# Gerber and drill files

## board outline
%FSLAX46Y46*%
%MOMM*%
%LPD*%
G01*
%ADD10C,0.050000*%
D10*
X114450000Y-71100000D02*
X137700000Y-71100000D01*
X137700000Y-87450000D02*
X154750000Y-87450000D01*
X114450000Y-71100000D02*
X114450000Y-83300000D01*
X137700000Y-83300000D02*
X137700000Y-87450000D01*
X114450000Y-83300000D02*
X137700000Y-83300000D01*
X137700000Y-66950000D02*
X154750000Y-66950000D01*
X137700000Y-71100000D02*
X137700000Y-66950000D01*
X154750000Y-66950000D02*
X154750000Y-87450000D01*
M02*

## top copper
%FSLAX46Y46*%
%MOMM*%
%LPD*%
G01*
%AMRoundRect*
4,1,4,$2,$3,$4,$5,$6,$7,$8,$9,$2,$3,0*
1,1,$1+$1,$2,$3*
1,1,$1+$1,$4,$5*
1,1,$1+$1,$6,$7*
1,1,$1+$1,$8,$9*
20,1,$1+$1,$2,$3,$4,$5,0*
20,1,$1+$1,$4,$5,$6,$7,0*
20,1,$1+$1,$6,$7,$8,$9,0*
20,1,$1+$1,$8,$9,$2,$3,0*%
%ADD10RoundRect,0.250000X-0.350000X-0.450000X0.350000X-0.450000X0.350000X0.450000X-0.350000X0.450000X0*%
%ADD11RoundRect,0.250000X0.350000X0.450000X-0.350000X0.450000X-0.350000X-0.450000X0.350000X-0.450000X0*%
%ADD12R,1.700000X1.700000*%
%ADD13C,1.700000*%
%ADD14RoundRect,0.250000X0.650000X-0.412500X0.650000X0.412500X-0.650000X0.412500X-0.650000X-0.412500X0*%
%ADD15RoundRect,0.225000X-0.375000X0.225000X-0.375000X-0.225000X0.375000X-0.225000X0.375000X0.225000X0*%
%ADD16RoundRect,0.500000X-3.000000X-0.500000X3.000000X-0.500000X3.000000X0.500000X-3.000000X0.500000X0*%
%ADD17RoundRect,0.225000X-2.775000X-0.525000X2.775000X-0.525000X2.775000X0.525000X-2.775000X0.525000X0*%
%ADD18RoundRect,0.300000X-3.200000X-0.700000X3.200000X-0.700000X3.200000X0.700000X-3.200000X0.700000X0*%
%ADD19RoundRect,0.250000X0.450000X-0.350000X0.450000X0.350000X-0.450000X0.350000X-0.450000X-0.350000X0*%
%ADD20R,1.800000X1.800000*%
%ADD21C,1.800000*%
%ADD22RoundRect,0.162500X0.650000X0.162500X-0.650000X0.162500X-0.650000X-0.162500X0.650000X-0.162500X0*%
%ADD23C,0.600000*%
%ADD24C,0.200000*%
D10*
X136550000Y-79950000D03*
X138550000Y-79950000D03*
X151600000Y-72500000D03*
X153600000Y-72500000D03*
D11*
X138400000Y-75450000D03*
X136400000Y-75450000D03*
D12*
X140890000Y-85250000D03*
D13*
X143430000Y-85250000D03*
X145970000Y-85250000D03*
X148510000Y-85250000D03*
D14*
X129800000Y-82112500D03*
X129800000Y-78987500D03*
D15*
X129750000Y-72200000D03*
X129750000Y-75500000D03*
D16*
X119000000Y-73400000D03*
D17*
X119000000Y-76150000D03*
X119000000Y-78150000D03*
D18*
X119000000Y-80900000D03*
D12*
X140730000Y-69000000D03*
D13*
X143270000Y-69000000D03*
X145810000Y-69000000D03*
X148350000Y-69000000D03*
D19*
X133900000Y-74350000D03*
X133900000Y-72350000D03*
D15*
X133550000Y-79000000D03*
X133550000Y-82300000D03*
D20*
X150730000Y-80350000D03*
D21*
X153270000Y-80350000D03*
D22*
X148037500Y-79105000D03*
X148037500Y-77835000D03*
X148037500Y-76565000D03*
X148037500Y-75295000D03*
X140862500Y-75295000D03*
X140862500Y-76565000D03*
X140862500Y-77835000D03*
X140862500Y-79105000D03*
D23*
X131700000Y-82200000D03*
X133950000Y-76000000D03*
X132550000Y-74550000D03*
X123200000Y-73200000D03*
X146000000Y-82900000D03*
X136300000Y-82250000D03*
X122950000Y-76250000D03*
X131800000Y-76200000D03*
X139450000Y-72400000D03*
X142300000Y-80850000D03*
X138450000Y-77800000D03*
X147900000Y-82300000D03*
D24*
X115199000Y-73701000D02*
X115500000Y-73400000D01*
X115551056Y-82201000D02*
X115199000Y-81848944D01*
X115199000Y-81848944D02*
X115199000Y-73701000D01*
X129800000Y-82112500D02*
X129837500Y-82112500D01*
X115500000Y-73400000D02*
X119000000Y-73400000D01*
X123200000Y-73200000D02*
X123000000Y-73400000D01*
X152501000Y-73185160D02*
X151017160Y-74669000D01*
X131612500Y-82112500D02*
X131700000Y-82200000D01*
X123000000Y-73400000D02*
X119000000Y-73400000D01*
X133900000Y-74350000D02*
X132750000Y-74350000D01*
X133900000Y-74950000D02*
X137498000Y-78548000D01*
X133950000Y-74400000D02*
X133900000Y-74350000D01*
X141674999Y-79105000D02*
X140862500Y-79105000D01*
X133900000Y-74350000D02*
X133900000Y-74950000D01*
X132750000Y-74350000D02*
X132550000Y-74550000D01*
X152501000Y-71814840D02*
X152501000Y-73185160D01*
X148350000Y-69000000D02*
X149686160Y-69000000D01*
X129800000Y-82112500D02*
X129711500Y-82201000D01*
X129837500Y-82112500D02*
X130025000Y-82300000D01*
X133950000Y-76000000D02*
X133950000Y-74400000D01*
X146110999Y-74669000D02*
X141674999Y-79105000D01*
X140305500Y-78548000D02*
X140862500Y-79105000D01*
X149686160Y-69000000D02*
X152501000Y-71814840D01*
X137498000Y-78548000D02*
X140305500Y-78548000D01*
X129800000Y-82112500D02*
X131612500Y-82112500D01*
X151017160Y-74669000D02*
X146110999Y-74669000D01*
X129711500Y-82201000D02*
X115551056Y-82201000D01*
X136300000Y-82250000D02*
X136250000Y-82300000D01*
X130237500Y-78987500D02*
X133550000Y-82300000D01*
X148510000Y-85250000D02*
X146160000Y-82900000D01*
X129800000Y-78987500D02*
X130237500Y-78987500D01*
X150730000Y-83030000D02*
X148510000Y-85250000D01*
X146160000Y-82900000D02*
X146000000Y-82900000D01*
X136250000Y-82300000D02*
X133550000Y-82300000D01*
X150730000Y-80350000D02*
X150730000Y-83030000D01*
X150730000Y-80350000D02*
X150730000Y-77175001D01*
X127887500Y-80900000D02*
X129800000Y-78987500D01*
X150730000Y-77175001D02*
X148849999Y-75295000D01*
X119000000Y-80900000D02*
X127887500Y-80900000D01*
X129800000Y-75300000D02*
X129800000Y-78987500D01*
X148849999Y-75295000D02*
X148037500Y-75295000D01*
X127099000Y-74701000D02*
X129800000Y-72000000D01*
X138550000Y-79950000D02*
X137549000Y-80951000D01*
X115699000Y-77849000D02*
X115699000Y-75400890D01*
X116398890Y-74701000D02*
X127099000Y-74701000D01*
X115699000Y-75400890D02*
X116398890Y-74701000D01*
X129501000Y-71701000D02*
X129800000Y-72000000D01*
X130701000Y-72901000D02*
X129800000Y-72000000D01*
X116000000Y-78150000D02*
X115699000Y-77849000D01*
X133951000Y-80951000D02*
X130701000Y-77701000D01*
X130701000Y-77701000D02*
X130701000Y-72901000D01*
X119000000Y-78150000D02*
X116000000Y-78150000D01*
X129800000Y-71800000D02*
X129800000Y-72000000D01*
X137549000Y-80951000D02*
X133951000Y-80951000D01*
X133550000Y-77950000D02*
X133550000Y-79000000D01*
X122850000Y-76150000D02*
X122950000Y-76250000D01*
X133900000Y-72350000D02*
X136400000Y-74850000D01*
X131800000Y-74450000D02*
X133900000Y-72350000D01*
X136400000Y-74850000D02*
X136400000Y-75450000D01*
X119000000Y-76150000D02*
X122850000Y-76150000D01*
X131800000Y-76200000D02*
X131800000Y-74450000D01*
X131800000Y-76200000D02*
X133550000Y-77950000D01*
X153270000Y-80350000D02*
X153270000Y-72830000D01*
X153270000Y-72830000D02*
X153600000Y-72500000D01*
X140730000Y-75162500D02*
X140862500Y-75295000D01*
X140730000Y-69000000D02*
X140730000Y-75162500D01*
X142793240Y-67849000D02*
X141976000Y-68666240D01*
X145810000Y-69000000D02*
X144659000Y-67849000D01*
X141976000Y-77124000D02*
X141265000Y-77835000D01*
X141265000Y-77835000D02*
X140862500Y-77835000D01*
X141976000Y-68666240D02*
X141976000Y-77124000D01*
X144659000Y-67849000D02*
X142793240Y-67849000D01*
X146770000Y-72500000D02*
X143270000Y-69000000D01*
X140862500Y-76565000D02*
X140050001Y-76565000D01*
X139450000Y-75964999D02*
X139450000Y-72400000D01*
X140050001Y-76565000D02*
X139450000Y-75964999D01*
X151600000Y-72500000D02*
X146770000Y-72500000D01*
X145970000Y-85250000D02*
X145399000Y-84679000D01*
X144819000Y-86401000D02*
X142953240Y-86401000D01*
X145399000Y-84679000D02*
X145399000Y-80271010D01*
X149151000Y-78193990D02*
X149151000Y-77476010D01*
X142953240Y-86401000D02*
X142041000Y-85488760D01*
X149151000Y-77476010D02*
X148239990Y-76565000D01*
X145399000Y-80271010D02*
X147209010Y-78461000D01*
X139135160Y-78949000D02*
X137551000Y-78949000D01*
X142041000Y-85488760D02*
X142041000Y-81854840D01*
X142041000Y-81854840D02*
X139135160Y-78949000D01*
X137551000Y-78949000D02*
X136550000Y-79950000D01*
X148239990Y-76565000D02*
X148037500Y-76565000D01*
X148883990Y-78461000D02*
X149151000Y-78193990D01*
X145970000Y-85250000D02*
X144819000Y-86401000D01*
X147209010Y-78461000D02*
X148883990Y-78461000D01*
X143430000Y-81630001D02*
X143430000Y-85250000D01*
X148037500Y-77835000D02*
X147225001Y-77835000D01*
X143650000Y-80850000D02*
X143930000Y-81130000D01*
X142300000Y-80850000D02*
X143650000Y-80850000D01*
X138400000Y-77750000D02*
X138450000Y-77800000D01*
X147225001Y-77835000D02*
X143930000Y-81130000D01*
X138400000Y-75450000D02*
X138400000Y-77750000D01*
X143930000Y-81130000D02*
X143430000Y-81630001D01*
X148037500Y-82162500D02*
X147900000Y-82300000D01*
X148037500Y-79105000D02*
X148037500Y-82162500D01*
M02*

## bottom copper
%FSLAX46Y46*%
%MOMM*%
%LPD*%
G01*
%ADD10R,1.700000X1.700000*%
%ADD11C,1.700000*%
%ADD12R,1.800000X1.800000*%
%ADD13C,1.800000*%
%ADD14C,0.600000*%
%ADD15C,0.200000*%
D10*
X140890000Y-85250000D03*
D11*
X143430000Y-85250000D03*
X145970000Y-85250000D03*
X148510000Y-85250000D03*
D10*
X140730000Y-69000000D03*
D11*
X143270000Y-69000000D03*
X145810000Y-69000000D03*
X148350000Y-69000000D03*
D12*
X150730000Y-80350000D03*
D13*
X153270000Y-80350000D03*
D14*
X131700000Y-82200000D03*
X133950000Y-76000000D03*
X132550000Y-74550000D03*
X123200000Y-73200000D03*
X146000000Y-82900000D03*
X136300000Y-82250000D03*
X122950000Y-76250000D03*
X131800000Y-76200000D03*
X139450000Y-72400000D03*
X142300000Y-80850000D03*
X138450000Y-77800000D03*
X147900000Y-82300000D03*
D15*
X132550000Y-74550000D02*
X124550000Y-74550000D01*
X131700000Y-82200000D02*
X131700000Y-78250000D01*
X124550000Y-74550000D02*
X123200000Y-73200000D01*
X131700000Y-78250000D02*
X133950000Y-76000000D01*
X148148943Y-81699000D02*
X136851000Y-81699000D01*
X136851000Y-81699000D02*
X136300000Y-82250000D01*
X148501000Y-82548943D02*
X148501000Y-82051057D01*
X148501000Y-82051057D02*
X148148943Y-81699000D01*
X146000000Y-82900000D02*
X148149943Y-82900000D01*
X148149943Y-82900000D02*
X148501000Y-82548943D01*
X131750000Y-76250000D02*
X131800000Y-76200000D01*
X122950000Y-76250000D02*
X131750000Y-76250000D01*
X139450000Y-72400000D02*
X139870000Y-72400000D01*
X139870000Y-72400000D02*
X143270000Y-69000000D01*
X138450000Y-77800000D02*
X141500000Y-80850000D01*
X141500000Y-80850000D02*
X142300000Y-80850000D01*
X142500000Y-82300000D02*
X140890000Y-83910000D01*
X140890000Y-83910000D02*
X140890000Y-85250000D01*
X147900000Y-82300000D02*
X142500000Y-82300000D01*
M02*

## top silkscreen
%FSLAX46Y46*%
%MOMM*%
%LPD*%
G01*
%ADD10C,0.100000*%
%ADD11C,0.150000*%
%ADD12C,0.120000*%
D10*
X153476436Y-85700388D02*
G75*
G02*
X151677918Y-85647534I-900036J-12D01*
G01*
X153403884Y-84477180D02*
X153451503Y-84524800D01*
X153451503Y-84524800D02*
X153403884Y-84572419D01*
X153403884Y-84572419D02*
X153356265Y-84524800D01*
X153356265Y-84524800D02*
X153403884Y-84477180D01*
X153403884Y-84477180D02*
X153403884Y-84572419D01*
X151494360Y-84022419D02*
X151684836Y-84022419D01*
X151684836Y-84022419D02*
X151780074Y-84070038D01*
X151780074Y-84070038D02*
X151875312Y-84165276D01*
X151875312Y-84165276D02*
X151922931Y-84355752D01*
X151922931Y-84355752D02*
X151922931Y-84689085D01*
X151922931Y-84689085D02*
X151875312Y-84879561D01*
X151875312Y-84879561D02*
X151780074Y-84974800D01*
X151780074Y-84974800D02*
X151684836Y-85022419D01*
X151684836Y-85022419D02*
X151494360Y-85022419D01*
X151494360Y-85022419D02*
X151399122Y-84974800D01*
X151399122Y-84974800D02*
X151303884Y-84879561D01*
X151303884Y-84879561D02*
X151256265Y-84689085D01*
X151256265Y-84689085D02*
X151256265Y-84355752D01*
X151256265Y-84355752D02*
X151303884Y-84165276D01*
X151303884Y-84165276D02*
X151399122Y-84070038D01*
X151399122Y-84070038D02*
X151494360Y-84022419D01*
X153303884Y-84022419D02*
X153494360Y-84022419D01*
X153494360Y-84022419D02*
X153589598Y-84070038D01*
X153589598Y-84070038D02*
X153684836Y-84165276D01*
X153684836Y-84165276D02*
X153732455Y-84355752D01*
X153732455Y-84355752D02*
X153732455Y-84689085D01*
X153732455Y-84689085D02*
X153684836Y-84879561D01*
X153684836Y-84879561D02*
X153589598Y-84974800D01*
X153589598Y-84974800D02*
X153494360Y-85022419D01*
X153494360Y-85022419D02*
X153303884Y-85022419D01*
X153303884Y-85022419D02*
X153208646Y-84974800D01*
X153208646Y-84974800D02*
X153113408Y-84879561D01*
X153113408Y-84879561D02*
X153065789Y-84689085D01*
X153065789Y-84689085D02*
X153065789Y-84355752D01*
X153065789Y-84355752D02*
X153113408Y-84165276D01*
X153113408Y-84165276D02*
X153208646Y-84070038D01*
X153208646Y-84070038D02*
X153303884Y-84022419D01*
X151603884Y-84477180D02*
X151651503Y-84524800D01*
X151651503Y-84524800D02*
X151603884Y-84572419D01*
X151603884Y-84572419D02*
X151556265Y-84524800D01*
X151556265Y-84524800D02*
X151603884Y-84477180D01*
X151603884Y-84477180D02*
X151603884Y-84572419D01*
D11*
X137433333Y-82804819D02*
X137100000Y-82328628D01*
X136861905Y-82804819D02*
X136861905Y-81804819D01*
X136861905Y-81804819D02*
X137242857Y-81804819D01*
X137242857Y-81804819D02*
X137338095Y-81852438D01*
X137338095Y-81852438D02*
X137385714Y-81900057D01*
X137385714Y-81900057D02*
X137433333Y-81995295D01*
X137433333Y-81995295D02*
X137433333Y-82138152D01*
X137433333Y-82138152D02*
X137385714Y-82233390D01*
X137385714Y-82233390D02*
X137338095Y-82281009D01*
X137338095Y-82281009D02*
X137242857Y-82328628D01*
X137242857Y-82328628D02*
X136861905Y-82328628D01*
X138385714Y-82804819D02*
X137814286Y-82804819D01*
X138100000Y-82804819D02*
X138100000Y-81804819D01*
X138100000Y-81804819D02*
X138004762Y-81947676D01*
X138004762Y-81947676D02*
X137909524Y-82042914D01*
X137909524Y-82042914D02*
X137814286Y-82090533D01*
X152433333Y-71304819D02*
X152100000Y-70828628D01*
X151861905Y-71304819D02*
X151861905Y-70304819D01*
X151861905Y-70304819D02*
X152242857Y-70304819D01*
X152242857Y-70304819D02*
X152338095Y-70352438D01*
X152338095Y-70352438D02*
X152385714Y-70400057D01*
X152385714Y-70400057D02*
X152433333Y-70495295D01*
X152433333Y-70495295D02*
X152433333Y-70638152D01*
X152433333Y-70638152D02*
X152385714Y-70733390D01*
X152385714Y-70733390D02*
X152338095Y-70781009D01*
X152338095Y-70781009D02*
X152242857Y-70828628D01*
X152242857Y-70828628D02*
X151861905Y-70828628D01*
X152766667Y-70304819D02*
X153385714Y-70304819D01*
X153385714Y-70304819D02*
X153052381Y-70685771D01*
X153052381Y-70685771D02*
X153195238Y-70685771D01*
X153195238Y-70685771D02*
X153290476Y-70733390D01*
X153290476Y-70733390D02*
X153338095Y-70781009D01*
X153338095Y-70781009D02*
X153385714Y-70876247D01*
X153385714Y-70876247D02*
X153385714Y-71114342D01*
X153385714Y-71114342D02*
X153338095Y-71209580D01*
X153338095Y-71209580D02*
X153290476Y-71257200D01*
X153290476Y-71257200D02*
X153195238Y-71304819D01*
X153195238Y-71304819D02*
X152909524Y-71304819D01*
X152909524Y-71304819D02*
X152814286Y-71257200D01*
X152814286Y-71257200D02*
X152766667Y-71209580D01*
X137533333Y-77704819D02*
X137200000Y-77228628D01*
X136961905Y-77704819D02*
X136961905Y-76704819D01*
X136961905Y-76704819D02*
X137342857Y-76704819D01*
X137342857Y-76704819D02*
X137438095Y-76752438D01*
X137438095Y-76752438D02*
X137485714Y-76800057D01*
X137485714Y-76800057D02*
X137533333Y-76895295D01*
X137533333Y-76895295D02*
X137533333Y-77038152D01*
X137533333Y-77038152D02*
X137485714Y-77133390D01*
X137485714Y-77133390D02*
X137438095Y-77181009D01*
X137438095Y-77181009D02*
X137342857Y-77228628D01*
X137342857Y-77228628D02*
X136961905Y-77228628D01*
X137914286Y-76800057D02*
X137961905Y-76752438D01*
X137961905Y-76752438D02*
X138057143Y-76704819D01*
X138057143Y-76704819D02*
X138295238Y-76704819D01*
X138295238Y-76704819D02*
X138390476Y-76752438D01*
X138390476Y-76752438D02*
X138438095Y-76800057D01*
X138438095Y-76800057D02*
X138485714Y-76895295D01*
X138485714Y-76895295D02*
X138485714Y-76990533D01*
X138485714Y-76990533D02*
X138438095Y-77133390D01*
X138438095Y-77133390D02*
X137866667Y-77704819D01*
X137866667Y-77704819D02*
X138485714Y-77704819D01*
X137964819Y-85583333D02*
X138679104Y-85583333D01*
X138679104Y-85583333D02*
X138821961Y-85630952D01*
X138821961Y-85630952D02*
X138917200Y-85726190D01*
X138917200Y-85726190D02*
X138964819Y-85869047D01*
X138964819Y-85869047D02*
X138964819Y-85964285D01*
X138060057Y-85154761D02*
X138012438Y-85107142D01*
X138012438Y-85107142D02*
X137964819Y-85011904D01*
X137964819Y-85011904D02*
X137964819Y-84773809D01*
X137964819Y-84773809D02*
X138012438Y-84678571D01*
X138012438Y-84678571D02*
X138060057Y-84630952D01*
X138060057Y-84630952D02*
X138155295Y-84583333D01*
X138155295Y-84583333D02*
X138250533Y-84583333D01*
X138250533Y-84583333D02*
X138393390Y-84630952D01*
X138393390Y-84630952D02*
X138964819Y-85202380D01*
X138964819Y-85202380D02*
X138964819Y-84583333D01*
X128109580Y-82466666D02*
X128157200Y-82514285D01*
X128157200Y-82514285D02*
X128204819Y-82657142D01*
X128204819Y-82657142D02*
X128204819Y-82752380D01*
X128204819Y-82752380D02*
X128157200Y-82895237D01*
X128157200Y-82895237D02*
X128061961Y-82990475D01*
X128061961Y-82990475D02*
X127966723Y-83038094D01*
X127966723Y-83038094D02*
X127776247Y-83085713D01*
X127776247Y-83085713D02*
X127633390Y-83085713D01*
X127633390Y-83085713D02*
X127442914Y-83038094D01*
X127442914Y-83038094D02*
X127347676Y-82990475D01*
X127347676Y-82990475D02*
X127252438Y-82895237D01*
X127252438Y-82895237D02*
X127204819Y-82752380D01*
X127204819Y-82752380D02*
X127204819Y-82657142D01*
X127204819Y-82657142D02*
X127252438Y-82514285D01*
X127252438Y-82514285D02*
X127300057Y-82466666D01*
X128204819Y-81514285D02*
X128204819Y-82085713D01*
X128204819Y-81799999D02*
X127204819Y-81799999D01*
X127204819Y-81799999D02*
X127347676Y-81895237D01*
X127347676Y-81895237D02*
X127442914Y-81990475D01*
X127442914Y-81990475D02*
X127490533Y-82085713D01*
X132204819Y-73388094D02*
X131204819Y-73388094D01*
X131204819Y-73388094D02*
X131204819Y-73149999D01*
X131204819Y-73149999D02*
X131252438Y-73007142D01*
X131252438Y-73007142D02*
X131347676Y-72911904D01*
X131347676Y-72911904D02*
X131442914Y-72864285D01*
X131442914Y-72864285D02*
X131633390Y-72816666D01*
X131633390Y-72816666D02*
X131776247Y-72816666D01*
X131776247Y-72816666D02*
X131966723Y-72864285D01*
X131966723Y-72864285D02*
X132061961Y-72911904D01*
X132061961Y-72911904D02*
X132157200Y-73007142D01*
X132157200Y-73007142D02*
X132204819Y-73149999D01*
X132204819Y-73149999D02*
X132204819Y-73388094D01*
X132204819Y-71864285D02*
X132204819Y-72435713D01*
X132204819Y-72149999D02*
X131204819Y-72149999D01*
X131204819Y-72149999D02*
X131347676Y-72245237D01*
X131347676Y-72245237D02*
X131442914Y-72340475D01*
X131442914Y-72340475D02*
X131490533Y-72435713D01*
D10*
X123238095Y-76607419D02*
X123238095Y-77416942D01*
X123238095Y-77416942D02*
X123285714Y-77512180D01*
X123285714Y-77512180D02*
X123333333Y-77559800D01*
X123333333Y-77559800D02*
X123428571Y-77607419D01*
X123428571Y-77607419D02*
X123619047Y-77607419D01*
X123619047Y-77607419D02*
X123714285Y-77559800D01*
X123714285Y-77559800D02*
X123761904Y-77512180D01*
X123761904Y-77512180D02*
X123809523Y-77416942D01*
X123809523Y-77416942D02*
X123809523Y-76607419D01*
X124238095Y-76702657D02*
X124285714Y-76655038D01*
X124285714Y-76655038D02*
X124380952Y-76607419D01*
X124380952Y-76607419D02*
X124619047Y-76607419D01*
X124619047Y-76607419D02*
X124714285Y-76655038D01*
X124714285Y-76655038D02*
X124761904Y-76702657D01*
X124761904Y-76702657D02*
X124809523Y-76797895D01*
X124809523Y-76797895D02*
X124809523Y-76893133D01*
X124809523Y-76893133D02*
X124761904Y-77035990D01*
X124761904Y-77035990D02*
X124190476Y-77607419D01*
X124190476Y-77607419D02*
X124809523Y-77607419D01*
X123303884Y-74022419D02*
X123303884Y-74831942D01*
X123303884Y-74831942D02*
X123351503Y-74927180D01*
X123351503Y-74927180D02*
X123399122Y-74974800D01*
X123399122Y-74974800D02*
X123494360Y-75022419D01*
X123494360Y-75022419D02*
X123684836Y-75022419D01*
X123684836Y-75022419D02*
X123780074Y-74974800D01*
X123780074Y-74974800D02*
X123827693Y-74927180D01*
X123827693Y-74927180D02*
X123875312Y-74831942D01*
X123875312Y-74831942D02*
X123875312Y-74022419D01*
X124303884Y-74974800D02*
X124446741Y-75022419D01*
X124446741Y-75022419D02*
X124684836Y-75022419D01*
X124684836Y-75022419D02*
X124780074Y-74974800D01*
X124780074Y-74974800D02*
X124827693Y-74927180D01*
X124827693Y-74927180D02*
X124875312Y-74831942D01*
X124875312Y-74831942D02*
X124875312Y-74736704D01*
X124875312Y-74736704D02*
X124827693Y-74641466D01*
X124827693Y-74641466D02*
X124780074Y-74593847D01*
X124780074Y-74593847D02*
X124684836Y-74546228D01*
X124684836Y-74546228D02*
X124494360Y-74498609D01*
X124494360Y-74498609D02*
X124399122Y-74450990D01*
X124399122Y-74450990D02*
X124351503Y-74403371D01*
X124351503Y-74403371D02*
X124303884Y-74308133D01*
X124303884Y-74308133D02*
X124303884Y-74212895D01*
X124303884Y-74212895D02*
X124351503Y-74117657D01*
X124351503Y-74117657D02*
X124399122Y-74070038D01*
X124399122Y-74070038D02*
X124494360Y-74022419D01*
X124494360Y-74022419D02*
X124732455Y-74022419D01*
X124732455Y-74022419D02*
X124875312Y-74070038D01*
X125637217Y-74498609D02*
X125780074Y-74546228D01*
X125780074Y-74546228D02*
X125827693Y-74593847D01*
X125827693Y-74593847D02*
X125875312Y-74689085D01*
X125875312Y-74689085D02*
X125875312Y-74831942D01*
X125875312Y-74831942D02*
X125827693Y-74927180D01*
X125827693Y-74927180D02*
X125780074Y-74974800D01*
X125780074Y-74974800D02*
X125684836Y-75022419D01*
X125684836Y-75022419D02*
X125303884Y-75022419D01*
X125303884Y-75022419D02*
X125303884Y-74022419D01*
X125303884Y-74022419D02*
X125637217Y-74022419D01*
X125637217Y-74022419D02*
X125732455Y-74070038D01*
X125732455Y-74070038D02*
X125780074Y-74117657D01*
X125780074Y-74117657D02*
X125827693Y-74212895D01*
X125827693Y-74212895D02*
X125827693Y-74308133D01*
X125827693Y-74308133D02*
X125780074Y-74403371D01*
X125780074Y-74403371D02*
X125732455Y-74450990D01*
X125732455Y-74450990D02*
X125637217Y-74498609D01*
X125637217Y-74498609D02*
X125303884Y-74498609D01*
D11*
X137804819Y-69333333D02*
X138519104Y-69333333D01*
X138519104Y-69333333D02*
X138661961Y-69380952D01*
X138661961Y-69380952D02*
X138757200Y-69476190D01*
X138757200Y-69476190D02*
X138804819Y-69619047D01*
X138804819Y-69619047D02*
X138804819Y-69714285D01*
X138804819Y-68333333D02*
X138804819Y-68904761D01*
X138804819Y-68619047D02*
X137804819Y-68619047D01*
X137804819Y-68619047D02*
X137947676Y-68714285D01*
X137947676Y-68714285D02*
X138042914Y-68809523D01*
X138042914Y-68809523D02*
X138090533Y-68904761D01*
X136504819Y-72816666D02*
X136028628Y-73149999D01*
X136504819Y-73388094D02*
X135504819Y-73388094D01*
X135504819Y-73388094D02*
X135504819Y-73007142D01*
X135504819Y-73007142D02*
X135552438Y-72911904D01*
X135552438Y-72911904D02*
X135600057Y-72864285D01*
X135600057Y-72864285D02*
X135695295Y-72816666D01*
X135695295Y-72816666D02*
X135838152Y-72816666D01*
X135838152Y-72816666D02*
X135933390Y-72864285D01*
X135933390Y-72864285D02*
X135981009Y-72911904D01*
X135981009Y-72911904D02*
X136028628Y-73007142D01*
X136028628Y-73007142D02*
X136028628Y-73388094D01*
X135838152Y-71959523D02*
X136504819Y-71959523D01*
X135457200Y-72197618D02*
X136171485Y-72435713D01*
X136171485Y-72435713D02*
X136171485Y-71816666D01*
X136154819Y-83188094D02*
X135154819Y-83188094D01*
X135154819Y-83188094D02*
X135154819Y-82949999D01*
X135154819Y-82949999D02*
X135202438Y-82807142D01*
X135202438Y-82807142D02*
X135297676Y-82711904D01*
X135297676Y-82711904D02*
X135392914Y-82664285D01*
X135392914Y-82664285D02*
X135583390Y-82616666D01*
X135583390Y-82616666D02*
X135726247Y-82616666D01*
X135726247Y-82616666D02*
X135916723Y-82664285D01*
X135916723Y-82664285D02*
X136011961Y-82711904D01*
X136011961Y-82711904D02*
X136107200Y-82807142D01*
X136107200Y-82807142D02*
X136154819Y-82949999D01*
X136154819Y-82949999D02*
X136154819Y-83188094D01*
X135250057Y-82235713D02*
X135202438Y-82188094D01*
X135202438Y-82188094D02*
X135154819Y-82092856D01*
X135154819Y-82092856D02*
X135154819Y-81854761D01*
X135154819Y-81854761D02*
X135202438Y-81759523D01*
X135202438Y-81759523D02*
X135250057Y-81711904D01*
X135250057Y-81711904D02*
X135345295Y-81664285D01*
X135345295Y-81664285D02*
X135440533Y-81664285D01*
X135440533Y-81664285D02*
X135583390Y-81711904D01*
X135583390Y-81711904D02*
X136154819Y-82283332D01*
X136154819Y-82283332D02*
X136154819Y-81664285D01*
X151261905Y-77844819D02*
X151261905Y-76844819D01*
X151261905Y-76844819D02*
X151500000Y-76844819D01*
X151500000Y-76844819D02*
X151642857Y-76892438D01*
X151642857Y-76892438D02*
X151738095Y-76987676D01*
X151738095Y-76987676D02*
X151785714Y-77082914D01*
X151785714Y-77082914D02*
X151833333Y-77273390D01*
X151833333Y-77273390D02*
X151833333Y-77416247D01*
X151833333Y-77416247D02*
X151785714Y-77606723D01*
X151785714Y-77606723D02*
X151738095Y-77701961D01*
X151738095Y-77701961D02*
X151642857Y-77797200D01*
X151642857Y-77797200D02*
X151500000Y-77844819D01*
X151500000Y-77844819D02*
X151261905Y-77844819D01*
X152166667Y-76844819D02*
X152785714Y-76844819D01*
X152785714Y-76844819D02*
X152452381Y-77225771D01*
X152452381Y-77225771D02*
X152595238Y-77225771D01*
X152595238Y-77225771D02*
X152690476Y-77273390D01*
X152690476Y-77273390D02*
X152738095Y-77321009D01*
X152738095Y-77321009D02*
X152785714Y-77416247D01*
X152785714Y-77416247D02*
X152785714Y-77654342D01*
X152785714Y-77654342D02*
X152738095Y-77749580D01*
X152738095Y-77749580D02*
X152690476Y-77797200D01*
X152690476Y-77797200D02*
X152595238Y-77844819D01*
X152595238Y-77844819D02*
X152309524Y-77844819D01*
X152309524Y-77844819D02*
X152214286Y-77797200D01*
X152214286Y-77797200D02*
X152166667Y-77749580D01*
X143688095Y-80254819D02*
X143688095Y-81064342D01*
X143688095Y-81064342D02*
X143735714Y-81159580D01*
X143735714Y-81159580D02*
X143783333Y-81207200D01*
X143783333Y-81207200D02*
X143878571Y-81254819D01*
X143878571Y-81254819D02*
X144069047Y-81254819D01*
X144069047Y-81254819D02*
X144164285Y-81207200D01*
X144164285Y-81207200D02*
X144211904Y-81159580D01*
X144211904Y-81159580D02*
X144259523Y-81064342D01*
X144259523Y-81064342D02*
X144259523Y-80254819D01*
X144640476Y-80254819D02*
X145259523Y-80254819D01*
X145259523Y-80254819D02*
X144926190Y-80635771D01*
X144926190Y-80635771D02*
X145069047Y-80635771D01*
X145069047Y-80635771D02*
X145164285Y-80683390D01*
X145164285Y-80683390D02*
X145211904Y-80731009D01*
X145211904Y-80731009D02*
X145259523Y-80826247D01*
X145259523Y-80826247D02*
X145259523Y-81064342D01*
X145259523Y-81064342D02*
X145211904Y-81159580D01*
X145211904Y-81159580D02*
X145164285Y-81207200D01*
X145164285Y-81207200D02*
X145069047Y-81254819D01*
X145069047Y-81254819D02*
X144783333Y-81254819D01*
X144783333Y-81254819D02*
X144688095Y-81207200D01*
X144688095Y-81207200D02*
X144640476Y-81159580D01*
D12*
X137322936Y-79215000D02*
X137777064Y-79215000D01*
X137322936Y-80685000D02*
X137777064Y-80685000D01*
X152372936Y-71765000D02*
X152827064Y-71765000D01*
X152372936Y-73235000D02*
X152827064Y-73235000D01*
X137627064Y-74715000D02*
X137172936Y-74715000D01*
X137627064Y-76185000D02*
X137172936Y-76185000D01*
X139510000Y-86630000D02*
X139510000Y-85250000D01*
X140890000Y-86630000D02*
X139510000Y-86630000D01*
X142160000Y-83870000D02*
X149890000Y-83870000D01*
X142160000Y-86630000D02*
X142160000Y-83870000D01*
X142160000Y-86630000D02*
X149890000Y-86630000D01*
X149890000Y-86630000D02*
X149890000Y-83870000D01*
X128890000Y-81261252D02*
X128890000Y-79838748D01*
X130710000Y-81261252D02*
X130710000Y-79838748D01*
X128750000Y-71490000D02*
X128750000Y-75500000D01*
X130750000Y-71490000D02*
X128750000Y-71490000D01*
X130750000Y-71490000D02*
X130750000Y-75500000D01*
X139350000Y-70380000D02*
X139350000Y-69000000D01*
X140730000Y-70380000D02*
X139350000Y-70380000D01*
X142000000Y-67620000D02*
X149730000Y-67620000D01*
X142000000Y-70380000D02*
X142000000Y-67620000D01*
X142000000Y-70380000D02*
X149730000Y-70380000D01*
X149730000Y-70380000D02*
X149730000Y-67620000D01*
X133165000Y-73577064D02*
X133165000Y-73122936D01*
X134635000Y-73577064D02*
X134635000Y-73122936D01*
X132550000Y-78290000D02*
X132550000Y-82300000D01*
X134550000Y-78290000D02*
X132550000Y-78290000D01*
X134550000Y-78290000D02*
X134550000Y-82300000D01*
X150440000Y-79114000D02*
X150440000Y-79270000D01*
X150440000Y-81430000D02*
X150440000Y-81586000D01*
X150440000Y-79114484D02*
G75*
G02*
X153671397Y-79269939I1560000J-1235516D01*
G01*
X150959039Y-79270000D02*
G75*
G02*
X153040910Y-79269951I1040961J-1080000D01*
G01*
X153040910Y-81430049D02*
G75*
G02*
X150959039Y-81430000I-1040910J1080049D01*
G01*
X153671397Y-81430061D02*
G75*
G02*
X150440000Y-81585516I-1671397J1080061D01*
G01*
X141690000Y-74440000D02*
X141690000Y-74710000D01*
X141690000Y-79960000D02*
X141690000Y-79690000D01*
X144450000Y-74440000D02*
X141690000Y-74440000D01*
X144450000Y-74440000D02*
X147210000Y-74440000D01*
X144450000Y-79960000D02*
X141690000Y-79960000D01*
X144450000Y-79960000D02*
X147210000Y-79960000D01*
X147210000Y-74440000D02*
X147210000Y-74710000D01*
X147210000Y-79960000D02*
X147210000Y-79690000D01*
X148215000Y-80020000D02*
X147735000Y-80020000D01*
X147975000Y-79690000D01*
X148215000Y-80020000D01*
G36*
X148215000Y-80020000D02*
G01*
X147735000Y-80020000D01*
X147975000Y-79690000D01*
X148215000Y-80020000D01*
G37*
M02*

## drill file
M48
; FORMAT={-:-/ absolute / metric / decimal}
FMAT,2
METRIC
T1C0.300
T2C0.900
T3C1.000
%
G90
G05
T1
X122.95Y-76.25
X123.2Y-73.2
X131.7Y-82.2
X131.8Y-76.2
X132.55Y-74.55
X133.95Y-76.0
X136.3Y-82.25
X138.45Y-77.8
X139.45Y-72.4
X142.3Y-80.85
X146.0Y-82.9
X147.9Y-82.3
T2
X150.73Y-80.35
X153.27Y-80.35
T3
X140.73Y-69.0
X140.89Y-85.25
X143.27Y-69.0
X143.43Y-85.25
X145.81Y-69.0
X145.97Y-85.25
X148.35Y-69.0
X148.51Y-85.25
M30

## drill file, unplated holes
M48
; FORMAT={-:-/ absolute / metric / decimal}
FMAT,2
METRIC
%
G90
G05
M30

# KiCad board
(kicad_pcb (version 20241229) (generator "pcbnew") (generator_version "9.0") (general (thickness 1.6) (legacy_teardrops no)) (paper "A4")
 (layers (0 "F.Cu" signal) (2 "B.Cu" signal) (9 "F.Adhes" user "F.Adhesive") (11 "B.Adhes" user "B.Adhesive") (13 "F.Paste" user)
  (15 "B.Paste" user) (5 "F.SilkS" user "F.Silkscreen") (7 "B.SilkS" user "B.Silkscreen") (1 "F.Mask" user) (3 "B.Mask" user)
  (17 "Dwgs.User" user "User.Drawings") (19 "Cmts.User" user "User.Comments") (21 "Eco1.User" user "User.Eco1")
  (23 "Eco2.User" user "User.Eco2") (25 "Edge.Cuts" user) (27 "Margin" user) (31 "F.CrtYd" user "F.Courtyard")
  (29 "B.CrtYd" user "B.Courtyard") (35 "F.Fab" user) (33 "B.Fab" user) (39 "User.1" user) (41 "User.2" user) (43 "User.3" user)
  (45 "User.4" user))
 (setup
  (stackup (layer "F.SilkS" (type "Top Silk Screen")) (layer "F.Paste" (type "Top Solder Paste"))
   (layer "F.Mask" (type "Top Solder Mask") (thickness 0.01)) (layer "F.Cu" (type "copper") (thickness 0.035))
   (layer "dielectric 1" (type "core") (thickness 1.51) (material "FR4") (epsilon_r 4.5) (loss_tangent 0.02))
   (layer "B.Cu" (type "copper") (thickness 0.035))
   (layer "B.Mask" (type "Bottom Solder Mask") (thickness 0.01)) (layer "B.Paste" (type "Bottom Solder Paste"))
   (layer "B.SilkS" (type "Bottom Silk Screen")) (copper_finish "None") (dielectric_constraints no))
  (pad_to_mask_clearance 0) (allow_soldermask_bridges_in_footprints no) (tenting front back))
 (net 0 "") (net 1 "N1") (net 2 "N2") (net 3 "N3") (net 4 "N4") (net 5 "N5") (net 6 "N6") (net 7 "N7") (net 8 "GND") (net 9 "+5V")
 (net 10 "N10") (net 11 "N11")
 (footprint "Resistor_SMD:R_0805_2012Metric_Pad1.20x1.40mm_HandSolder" (layer "F.Cu") (at 137.55 79.95)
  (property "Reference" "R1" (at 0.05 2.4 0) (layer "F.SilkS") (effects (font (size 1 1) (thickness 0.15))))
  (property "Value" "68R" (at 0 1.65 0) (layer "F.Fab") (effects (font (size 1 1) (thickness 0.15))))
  (fp_line (start -0.227064 -0.735) (end 0.227064 -0.735) (stroke (width 0.12) (type solid)) (layer "F.SilkS"))
  (fp_line (start -0.227064 0.735) (end 0.227064 0.735) (stroke (width 0.12) (type solid)) (layer "F.SilkS"))
  (pad "1" smd roundrect (at -1 0) (size 1.2 1.4) (layers "F.Cu" "F.Mask" "F.Paste") (roundrect_rratio 0.208333) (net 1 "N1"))
  (pad "2" smd roundrect (at 1 0) (size 1.2 1.4) (layers "F.Cu" "F.Mask" "F.Paste") (roundrect_rratio 0.208333) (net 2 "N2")))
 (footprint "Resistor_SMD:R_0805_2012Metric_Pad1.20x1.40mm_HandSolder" (layer "F.Cu") (at 152.6 72.5)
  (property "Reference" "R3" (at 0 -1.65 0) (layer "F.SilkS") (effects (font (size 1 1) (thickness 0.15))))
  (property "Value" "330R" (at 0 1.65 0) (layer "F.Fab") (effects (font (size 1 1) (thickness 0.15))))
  (fp_line (start -0.227064 -0.735) (end 0.227064 -0.735) (stroke (width 0.12) (type solid)) (layer "F.SilkS"))
  (fp_line (start -0.227064 0.735) (end 0.227064 0.735) (stroke (width 0.12) (type solid)) (layer "F.SilkS"))
  (pad "1" smd roundrect (at -1 0) (size 1.2 1.4) (layers "F.Cu" "F.Mask" "F.Paste") (roundrect_rratio 0.208333) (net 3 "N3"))
  (pad "2" smd roundrect (at 1 0) (size 1.2 1.4) (layers "F.Cu" "F.Mask" "F.Paste") (roundrect_rratio 0.208333) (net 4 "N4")))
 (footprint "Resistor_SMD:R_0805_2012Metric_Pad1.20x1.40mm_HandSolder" (layer "F.Cu") (at 137.4 75.45 180)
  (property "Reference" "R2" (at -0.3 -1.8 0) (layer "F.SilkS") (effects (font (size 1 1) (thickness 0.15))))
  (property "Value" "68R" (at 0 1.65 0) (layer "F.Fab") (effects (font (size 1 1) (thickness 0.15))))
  (fp_line (start -0.227064 0.735) (end 0.227064 0.735) (stroke (width 0.12) (type solid)) (layer "F.SilkS"))
  (fp_line (start -0.227064 -0.735) (end 0.227064 -0.735) (stroke (width 0.12) (type solid)) (layer "F.SilkS"))
  (pad "1" smd roundrect (at -1 0 180) (size 1.2 1.4) (layers "F.Cu" "F.Mask" "F.Paste") (roundrect_rratio 0.208333) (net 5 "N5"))
  (pad "2" smd roundrect (at 1 0 180) (size 1.2 1.4) (layers "F.Cu" "F.Mask" "F.Paste") (roundrect_rratio 0.208333) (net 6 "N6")))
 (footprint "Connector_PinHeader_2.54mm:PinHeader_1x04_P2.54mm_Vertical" (layer "F.Cu") (at 140.89 85.25 90)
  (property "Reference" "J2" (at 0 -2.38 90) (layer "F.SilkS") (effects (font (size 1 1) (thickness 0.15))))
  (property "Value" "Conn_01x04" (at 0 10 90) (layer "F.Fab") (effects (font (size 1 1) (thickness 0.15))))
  (fp_line (start -1.38 -1.38) (end 0 -1.38) (stroke (width 0.12) (type solid)) (layer "F.SilkS"))
  (fp_line (start -1.38 0) (end -1.38 -1.38) (stroke (width 0.12) (type solid)) (layer "F.SilkS"))
  (fp_line (start 1.38 1.27) (end 1.38 9) (stroke (width 0.12) (type solid)) (layer "F.SilkS"))
  (fp_line (start -1.38 1.27) (end 1.38 1.27) (stroke (width 0.12) (type solid)) (layer "F.SilkS"))
  (fp_line (start -1.38 1.27) (end -1.38 9) (stroke (width 0.12) (type solid)) (layer "F.SilkS"))
  (fp_line (start -1.38 9) (end 1.38 9) (stroke (width 0.12) (type solid)) (layer "F.SilkS"))
  (pad "1" thru_hole rect (at 0 0 90) (size 1.7 1.7) (drill 1) (layers "*.Cu" "*.Mask") (remove_unused_layers no) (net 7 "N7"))
  (pad "2" thru_hole circle (at 0 2.54 90) (size 1.7 1.7) (drill 1) (layers "*.Cu" "*.Mask") (remove_unused_layers no) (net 5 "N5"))
  (pad "3" thru_hole circle (at 0 5.08 90) (size 1.7 1.7) (drill 1) (layers "*.Cu" "*.Mask") (remove_unused_layers no) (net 1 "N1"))
  (pad "4" thru_hole circle (at 0 7.62 90) (size 1.7 1.7) (drill 1) (layers "*.Cu" "*.Mask") (remove_unused_layers no) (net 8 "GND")))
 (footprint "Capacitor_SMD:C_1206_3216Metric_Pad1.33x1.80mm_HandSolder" (layer "F.Cu") (at 129.8 80.55 90)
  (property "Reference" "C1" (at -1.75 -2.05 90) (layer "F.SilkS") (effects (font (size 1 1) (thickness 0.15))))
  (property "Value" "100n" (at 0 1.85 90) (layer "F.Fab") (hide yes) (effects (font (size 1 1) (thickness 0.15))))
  (fp_line (start -0.711252 -0.91) (end 0.711252 -0.91) (stroke (width 0.12) (type solid)) (layer "F.SilkS"))
  (fp_line (start -0.711252 0.91) (end 0.711252 0.91) (stroke (width 0.12) (type solid)) (layer "F.SilkS"))
  (pad "1" smd roundrect (at -1.5625 0 90) (size 1.325 1.8) (layers "F.Cu" "F.Mask" "F.Paste") (roundrect_rratio 0.188679) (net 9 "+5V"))
  (pad "2" smd roundrect (at 1.5625 0 90) (size 1.325 1.8) (layers "F.Cu" "F.Mask" "F.Paste") (roundrect_rratio 0.188679) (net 8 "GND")))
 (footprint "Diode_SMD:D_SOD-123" (layer "F.Cu") (at 129.75 73.85 -90)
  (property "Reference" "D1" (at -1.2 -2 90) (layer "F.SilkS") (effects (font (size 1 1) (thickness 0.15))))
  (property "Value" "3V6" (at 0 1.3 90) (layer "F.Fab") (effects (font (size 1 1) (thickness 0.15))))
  (fp_line (start -2.36 1) (end 1.65 1) (stroke (width 0.12) (type solid)) (layer "F.SilkS"))
  (fp_line (start -2.36 -1) (end -2.36 1) (stroke (width 0.12) (type solid)) (layer "F.SilkS"))
  (fp_line (start -2.36 -1) (end 1.65 -1) (stroke (width 0.12) (type solid)) (layer "F.SilkS"))
  (pad "1" smd roundrect (at -1.65 0 270) (size 0.9 1.2) (layers "F.Cu" "F.Mask" "F.Paste") (roundrect_rratio 0.25) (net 2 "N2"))
  (pad "2" smd roundrect (at 1.65 0 270) (size 0.9 1.2) (layers "F.Cu" "F.Mask" "F.Paste") (roundrect_rratio 0.25) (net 8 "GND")))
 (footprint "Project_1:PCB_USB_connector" (layer "F.Cu") (at 119 77.15)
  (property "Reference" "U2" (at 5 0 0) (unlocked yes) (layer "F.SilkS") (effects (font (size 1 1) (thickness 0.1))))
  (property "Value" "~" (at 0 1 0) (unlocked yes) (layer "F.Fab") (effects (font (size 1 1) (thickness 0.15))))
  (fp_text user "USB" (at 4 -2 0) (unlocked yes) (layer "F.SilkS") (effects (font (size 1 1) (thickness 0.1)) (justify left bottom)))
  (pad "1" smd roundrect (at 0 -3.75) (size 7 2) (layers "F.Cu" "F.Mask" "F.Paste") (roundrect_rratio 0.25) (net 9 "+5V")
   (thermal_bridge_angle 45))
  (pad "2" smd roundrect (at 0 -1) (size 6 1.5) (layers "F.Cu" "F.Mask" "F.Paste") (roundrect_rratio 0.15) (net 6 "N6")
   (thermal_bridge_angle 45))
  (pad "3" smd roundrect (at 0 1) (size 6 1.5) (layers "F.Cu" "F.Mask" "F.Paste") (roundrect_rratio 0.15) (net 2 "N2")
   (thermal_bridge_angle 45))
  (pad "4" smd roundrect (at 0 3.75) (size 7 2) (layers "F.Cu" "F.Mask" "F.Paste") (roundrect_rratio 0.15) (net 8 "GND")
   (thermal_bridge_angle 45)))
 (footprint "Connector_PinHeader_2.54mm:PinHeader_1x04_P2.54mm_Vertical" (layer "F.Cu") (at 140.73 69 90)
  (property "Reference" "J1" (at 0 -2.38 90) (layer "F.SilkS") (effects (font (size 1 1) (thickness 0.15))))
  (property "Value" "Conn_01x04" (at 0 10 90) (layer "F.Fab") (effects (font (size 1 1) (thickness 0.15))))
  (fp_line (start -1.38 -1.38) (end 0 -1.38) (stroke (width 0.12) (type solid)) (layer "F.SilkS"))
  (fp_line (start -1.38 0) (end -1.38 -1.38) (stroke (width 0.12) (type solid)) (layer "F.SilkS"))
  (fp_line (start 1.38 1.27) (end 1.38 9) (stroke (width 0.12) (type solid)) (layer "F.SilkS"))
  (fp_line (start -1.38 1.27) (end 1.38 1.27) (stroke (width 0.12) (type solid)) (layer "F.SilkS"))
  (fp_line (start -1.38 1.27) (end -1.38 9) (stroke (width 0.12) (type solid)) (layer "F.SilkS"))
  (fp_line (start -1.38 9) (end 1.38 9) (stroke (width 0.12) (type solid)) (layer "F.SilkS"))
  (pad "1" thru_hole rect (at 0 0 90) (size 1.7 1.7) (drill 1) (layers "*.Cu" "*.Mask") (remove_unused_layers no) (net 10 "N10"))
  (pad "2" thru_hole circle (at 0 2.54 90) (size 1.7 1.7) (drill 1) (layers "*.Cu" "*.Mask") (remove_unused_layers no) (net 3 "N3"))
  (pad "3" thru_hole circle (at 0 5.08 90) (size 1.7 1.7) (drill 1) (layers "*.Cu" "*.Mask") (remove_unused_layers no) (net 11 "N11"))
  (pad "4" thru_hole circle (at 0 7.62 90) (size 1.7 1.7) (drill 1) (layers "*.Cu" "*.Mask") (remove_unused_layers no) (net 9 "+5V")))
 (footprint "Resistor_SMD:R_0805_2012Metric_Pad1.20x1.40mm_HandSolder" (layer "F.Cu") (at 133.9 73.35 90)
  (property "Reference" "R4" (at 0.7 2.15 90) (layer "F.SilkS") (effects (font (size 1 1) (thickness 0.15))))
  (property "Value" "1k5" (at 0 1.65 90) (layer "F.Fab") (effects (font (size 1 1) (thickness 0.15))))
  (fp_line (start -0.227064 -0.735) (end 0.227064 -0.735) (stroke (width 0.12) (type solid)) (layer "F.SilkS"))
  (fp_line (start -0.227064 0.735) (end 0.227064 0.735) (stroke (width 0.12) (type solid)) (layer "F.SilkS"))
  (pad "1" smd roundrect (at -1 0 90) (size 1.2 1.4) (layers "F.Cu" "F.Mask" "F.Paste") (roundrect_rratio 0.208333) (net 9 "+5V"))
  (pad "2" smd roundrect (at 1 0 90) (size 1.2 1.4) (layers "F.Cu" "F.Mask" "F.Paste") (roundrect_rratio 0.208333) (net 6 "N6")))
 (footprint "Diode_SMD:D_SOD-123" (layer "F.Cu") (at 133.55 80.65 -90)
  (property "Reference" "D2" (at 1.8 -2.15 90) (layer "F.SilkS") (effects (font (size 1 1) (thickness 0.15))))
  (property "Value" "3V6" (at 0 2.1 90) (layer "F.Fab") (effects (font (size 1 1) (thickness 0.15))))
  (fp_line (start -2.36 1) (end 1.65 1) (stroke (width 0.12) (type solid)) (layer "F.SilkS"))
  (fp_line (start -2.36 -1) (end -2.36 1) (stroke (width 0.12) (type solid)) (layer "F.SilkS"))
  (fp_line (start -2.36 -1) (end 1.65 -1) (stroke (width 0.12) (type solid)) (layer "F.SilkS"))
  (pad "1" smd roundrect (at -1.65 0 270) (size 0.9 1.2) (layers "F.Cu" "F.Mask" "F.Paste") (roundrect_rratio 0.25) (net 6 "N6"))
  (pad "2" smd roundrect (at 1.65 0 270) (size 0.9 1.2) (layers "F.Cu" "F.Mask" "F.Paste") (roundrect_rratio 0.25) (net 8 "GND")))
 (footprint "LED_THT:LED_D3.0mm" (layer "F.Cu") (at 150.73 80.35)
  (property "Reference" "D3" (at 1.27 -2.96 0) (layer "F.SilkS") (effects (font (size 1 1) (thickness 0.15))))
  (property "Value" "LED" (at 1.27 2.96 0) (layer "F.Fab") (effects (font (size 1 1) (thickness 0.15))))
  (fp_line (start -0.29 -1.236) (end -0.29 -1.08) (stroke (width 0.12) (type solid)) (layer "F.SilkS"))
  (fp_line (start -0.29 1.08) (end -0.29 1.236) (stroke (width 0.12) (type solid)) (layer "F.SilkS"))
  (fp_arc (start -0.29 -1.235516) (mid 1.365624 -1.987701) (end 2.941397 -1.080061) (stroke (width 0.12) (type solid)) (layer "F.SilkS"))
  (fp_arc (start 0.229039 -1.08) (mid 1.269964 -1.5) (end 2.31091 -1.080049) (stroke (width 0.12) (type solid)) (layer "F.SilkS"))
  (fp_arc (start 2.31091 1.080049) (mid 1.269964 1.5) (end 0.229039 1.08) (stroke (width 0.12) (type solid)) (layer "F.SilkS"))
  (fp_arc (start 2.941397 1.080061) (mid 1.365624 1.987701) (end -0.29 1.235516) (stroke (width 0.12) (type solid)) (layer "F.SilkS"))
  (pad "1" thru_hole rect (at 0 0) (size 1.8 1.8) (drill 0.9) (layers "*.Cu" "*.Mask") (remove_unused_layers no) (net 8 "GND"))
  (pad "2" thru_hole circle (at 2.54 0) (size 1.8 1.8) (drill 0.9) (layers "*.Cu" "*.Mask") (remove_unused_layers no) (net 4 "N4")))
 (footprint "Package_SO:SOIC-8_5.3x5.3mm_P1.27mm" (layer "F.Cu") (at 144.45 77.2 180)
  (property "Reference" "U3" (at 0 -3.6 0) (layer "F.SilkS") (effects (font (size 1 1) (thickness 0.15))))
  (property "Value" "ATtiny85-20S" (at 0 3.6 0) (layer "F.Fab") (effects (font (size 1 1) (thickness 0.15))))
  (fp_line (start 2.76 2.76) (end 2.76 2.49) (stroke (width 0.12) (type solid)) (layer "F.SilkS"))
  (fp_line (start 2.76 -2.76) (end 2.76 -2.49) (stroke (width 0.12) (type solid)) (layer "F.SilkS"))
  (fp_line (start 0 2.76) (end 2.76 2.76) (stroke (width 0.12) (type solid)) (layer "F.SilkS"))
  (fp_line (start 0 2.76) (end -2.76 2.76) (stroke (width 0.12) (type solid)) (layer "F.SilkS"))
  (fp_line (start 0 -2.76) (end 2.76 -2.76) (stroke (width 0.12) (type solid)) (layer "F.SilkS"))
  (fp_line (start 0 -2.76) (end -2.76 -2.76) (stroke (width 0.12) (type solid)) (layer "F.SilkS"))
  (fp_line (start -2.76 2.76) (end -2.76 2.49) (stroke (width 0.12) (type solid)) (layer "F.SilkS"))
  (fp_line (start -2.76 -2.76) (end -2.76 -2.49) (stroke (width 0.12) (type solid)) (layer "F.SilkS"))
  (fp_poly (pts (xy -3.525 -2.49) (xy -3.765 -2.82) (xy -3.285 -2.82)) (stroke (width 0.12) (type solid)) (fill yes) (layer "F.SilkS"))
  (pad "1" smd roundrect (at -3.5875 -1.905 180) (size 1.625 0.65) (layers "F.Cu" "F.Mask" "F.Paste") (roundrect_rratio 0.25) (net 7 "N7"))
  (pad "2" smd roundrect (at -3.5875 -0.635 180) (size 1.625 0.65) (layers "F.Cu" "F.Mask" "F.Paste") (roundrect_rratio 0.25) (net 5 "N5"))
  (pad "3" smd roundrect (at -3.5875 0.635 180) (size 1.625 0.65) (layers "F.Cu" "F.Mask" "F.Paste") (roundrect_rratio 0.25) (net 1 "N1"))
  (pad "4" smd roundrect (at -3.5875 1.905 180) (size 1.625 0.65) (layers "F.Cu" "F.Mask" "F.Paste") (roundrect_rratio 0.25) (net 8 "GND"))
  (pad "5" smd roundrect (at 3.5875 1.905 180) (size 1.625 0.65) (layers "F.Cu" "F.Mask" "F.Paste") (roundrect_rratio 0.25) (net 10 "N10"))
  (pad "6" smd roundrect (at 3.5875 0.635 180) (size 1.625 0.65) (layers "F.Cu" "F.Mask" "F.Paste") (roundrect_rratio 0.25) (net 3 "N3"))
  (pad "7" smd roundrect (at 3.5875 -0.635 180) (size 1.625 0.65) (layers "F.Cu" "F.Mask" "F.Paste") (roundrect_rratio 0.25) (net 11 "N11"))
  (pad "8" smd roundrect (at 3.5875 -1.905 180) (size 1.625 0.65) (layers "F.Cu" "F.Mask" "F.Paste") (roundrect_rratio 0.25) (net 9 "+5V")))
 (gr_arc (start 153.476436 85.700388) (mid 152.55 86.6) (end 151.677989 85.647538) (stroke (width 0.1) (type default)) (layer "F.SilkS"))
 (gr_line (start 114.45 71.1) (end 137.7 71.1) (stroke (width 0.05) (type default)) (layer "Edge.Cuts"))
 (gr_line (start 137.7 87.45) (end 154.75 87.45) (stroke (width 0.05) (type solid)) (layer "Edge.Cuts"))
 (gr_line (start 114.45 71.1) (end 114.45 83.3) (stroke (width 0.05) (type solid)) (layer "Edge.Cuts"))
 (gr_line (start 137.7 83.3) (end 137.7 87.45) (stroke (width 0.05) (type default)) (layer "Edge.Cuts"))
 (gr_line (start 114.45 83.3) (end 137.7 83.3) (stroke (width 0.05) (type default)) (layer "Edge.Cuts"))
 (gr_line (start 137.7 66.95) (end 154.75 66.95) (stroke (width 0.05) (type default)) (layer "Edge.Cuts"))
 (gr_line (start 137.7 71.1) (end 137.7 66.95) (stroke (width 0.05) (type default)) (layer "Edge.Cuts"))
 (gr_line (start 154.75 66.95) (end 154.75 87.45) (stroke (width 0.05) (type default)) (layer "Edge.Cuts"))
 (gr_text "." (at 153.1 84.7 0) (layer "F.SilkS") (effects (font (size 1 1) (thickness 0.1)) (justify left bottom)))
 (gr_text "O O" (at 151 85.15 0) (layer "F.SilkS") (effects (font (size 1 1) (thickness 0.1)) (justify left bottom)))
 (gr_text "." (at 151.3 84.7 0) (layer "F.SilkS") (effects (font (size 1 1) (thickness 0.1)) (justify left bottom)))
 (segment (start 115.199 73.701) (end 115.5 73.4) (width 0.2) (layer "F.Cu") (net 9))
 (segment (start 115.551056 82.201) (end 115.199 81.848944) (width 0.2) (layer "F.Cu") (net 9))
 (segment (start 115.199 81.848944) (end 115.199 73.701) (width 0.2) (layer "F.Cu") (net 9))
 (segment (start 129.8 82.1125) (end 129.8375 82.1125) (width 0.2) (layer "F.Cu") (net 9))
 (segment (start 115.5 73.4) (end 119 73.4) (width 0.2) (layer "F.Cu") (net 9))
 (segment (start 123.2 73.2) (end 123 73.4) (width 0.2) (layer "F.Cu") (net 9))
 (segment (start 152.501 73.18516) (end 151.01716 74.669) (width 0.2) (layer "F.Cu") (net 9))
 (segment (start 131.6125 82.1125) (end 131.7 82.2) (width 0.2) (layer "F.Cu") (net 9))
 (segment (start 123 73.4) (end 119 73.4) (width 0.2) (layer "F.Cu") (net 9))
 (segment (start 133.9 74.35) (end 132.75 74.35) (width 0.2) (layer "F.Cu") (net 9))
 (segment (start 133.9 74.95) (end 137.498 78.548) (width 0.2) (layer "F.Cu") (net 9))
 (segment (start 133.95 74.4) (end 133.9 74.35) (width 0.2) (layer "F.Cu") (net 9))
 (segment (start 141.674999 79.105) (end 140.8625 79.105) (width 0.2) (layer "F.Cu") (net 9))
 (segment (start 133.9 74.35) (end 133.9 74.95) (width 0.2) (layer "F.Cu") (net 9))
 (segment (start 132.75 74.35) (end 132.55 74.55) (width 0.2) (layer "F.Cu") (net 9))
 (segment (start 152.501 71.81484) (end 152.501 73.18516) (width 0.2) (layer "F.Cu") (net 9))
 (segment (start 148.35 69) (end 149.68616 69) (width 0.2) (layer "F.Cu") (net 9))
 (segment (start 129.8 82.1125) (end 129.7115 82.201) (width 0.2) (layer "F.Cu") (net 9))
 (segment (start 129.8375 82.1125) (end 130.025 82.3) (width 0.2) (layer "F.Cu") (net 9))
 (segment (start 133.95 76) (end 133.95 74.4) (width 0.2) (layer "F.Cu") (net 9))
 (segment (start 146.110999 74.669) (end 141.674999 79.105) (width 0.2) (layer "F.Cu") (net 9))
 (segment (start 140.3055 78.548) (end 140.8625 79.105) (width 0.2) (layer "F.Cu") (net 9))
 (segment (start 149.68616 69) (end 152.501 71.81484) (width 0.2) (layer "F.Cu") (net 9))
 (segment (start 137.498 78.548) (end 140.3055 78.548) (width 0.2) (layer "F.Cu") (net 9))
 (segment (start 129.8 82.1125) (end 131.6125 82.1125) (width 0.2) (layer "F.Cu") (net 9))
 (segment (start 151.01716 74.669) (end 146.110999 74.669) (width 0.2) (layer "F.Cu") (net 9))
 (segment (start 129.7115 82.201) (end 115.551056 82.201) (width 0.2) (layer "F.Cu") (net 9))
 (via (at 131.7 82.2) (size 0.6) (drill 0.3) (layers "F.Cu" "B.Cu") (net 9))
 (via (at 133.95 76) (size 0.6) (drill 0.3) (layers "F.Cu" "B.Cu") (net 9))
 (via (at 132.55 74.55) (size 0.6) (drill 0.3) (layers "F.Cu" "B.Cu") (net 9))
 (via (at 123.2 73.2) (size 0.6) (drill 0.3) (layers "F.Cu" "B.Cu") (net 9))
 (segment (start 132.55 74.55) (end 124.55 74.55) (width 0.2) (layer "B.Cu") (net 9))
 (segment (start 131.7 82.2) (end 131.7 78.25) (width 0.2) (layer "B.Cu") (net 9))
 (segment (start 124.55 74.55) (end 123.2 73.2) (width 0.2) (layer "B.Cu") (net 9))
 (segment (start 131.7 78.25) (end 133.95 76) (width 0.2) (layer "B.Cu") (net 9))
 (segment (start 136.3 82.25) (end 136.25 82.3) (width 0.2) (layer "F.Cu") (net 8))
 (segment (start 130.2375 78.9875) (end 133.55 82.3) (width 0.2) (layer "F.Cu") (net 8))
 (segment (start 148.51 85.25) (end 146.16 82.9) (width 0.2) (layer "F.Cu") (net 8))
 (segment (start 129.8 78.9875) (end 130.2375 78.9875) (width 0.2) (layer "F.Cu") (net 8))
 (segment (start 150.73 83.03) (end 148.51 85.25) (width 0.2) (layer "F.Cu") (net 8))
 (segment (start 146.16 82.9) (end 146 82.9) (width 0.2) (layer "F.Cu") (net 8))
 (segment (start 136.25 82.3) (end 133.55 82.3) (width 0.2) (layer "F.Cu") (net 8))
 (segment (start 150.73 80.35) (end 150.73 83.03) (width 0.2) (layer "F.Cu") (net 8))
 (segment (start 150.73 80.35) (end 150.73 77.175001) (width 0.2) (layer "F.Cu") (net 8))
 (segment (start 127.8875 80.9) (end 129.8 78.9875) (width 0.2) (layer "F.Cu") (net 8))
 (segment (start 150.73 77.175001) (end 148.849999 75.295) (width 0.2) (layer "F.Cu") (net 8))
 (segment (start 119 80.9) (end 127.8875 80.9) (width 0.2) (layer "F.Cu") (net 8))
 (segment (start 129.8 75.3) (end 129.8 78.9875) (width 0.2) (layer "F.Cu") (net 8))
 (segment (start 148.849999 75.295) (end 148.0375 75.295) (width 0.2) (layer "F.Cu") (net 8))
 (via (at 146 82.9) (size 0.6) (drill 0.3) (layers "F.Cu" "B.Cu") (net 8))
 (via (at 136.3 82.25) (size 0.6) (drill 0.3) (layers "F.Cu" "B.Cu") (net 8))
 (segment (start 148.148943 81.699) (end 136.851 81.699) (width 0.2) (layer "B.Cu") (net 8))
 (segment (start 136.851 81.699) (end 136.3 82.25) (width 0.2) (layer "B.Cu") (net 8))
 (segment (start 148.501 82.548943) (end 148.501 82.051057) (width 0.2) (layer "B.Cu") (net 8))
 (segment (start 148.501 82.051057) (end 148.148943 81.699) (width 0.2) (layer "B.Cu") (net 8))
 (segment (start 146 82.9) (end 148.149943 82.9) (width 0.2) (layer "B.Cu") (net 8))
 (segment (start 148.149943 82.9) (end 148.501 82.548943) (width 0.2) (layer "B.Cu") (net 8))
 (segment (start 127.099 74.701) (end 129.8 72) (width 0.2) (layer "F.Cu") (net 2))
 (segment (start 138.55 79.95) (end 137.549 80.951) (width 0.2) (layer "F.Cu") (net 2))
 (segment (start 115.699 77.849) (end 115.699 75.40089) (width 0.2) (layer "F.Cu") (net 2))
 (segment (start 116.39889 74.701) (end 127.099 74.701) (width 0.2) (layer "F.Cu") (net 2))
 (segment (start 115.699 75.40089) (end 116.39889 74.701) (width 0.2) (layer "F.Cu") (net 2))
 (segment (start 129.501 71.701) (end 129.8 72) (width 0.2) (layer "F.Cu") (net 2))
 (segment (start 130.701 72.901) (end 129.8 72) (width 0.2) (layer "F.Cu") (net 2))
 (segment (start 116 78.15) (end 115.699 77.849) (width 0.2) (layer "F.Cu") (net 2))
 (segment (start 133.951 80.951) (end 130.701 77.701) (width 0.2) (layer "F.Cu") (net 2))
 (segment (start 130.701 77.701) (end 130.701 72.901) (width 0.2) (layer "F.Cu") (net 2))
 (segment (start 119 78.15) (end 116 78.15) (width 0.2) (layer "F.Cu") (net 2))
 (segment (start 129.8 71.8) (end 129.8 72) (width 0.2) (layer "F.Cu") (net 2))
 (segment (start 137.549 80.951) (end 133.951 80.951) (width 0.2) (layer "F.Cu") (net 2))
 (segment (start 133.55 77.95) (end 133.55 79) (width 0.2) (layer "F.Cu") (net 6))
 (segment (start 122.85 76.15) (end 122.95 76.25) (width 0.2) (layer "F.Cu") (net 6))
 (segment (start 133.9 72.35) (end 136.4 74.85) (width 0.2) (layer "F.Cu") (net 6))
 (segment (start 131.8 74.45) (end 133.9 72.35) (width 0.2) (layer "F.Cu") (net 6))
 (segment (start 136.4 74.85) (end 136.4 75.45) (width 0.2) (layer "F.Cu") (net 6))
 (segment (start 119 76.15) (end 122.85 76.15) (width 0.2) (layer "F.Cu") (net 6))
 (segment (start 131.8 76.2) (end 131.8 74.45) (width 0.2) (layer "F.Cu") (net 6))
 (segment (start 131.8 76.2) (end 133.55 77.95) (width 0.2) (layer "F.Cu") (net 6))
 (via (at 122.95 76.25) (size 0.6) (drill 0.3) (layers "F.Cu" "B.Cu") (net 6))
 (via (at 131.8 76.2) (size 0.6) (drill 0.3) (layers "F.Cu" "B.Cu") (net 6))
 (segment (start 131.75 76.25) (end 131.8 76.2) (width 0.2) (layer "B.Cu") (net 6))
 (segment (start 122.95 76.25) (end 131.75 76.25) (width 0.2) (layer "B.Cu") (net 6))
 (segment (start 153.27 80.35) (end 153.27 72.83) (width 0.2) (layer "F.Cu") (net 4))
 (segment (start 153.27 72.83) (end 153.6 72.5) (width 0.2) (layer "F.Cu") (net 4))
 (segment (start 140.73 75.1625) (end 140.8625 75.295) (width 0.2) (layer "F.Cu") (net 10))
 (segment (start 140.73 69) (end 140.73 75.1625) (width 0.2) (layer "F.Cu") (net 10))
 (segment (start 142.79324 67.849) (end 141.976 68.66624) (width 0.2) (layer "F.Cu") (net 11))
 (segment (start 145.81 69) (end 144.659 67.849) (width 0.2) (layer "F.Cu") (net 11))
 (segment (start 141.976 77.124) (end 141.265 77.835) (width 0.2) (layer "F.Cu") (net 11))
 (segment (start 141.265 77.835) (end 140.8625 77.835) (width 0.2) (layer "F.Cu") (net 11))
 (segment (start 141.976 68.66624) (end 141.976 77.124) (width 0.2) (layer "F.Cu") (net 11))
 (segment (start 144.659 67.849) (end 142.79324 67.849) (width 0.2) (layer "F.Cu") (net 11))
 (segment (start 146.77 72.5) (end 143.27 69) (width 0.2) (layer "F.Cu") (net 3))
 (segment (start 140.8625 76.565) (end 140.050001 76.565) (width 0.2) (layer "F.Cu") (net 3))
 (segment (start 139.45 75.964999) (end 139.45 72.4) (width 0.2) (layer "F.Cu") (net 3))
 (segment (start 140.050001 76.565) (end 139.45 75.964999) (width 0.2) (layer "F.Cu") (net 3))
 (segment (start 151.6 72.5) (end 146.77 72.5) (width 0.2) (layer "F.Cu") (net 3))
 (via (at 139.45 72.4) (size 0.6) (drill 0.3) (layers "F.Cu" "B.Cu") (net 3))
 (segment (start 139.45 72.4) (end 139.87 72.4) (width 0.2) (layer "B.Cu") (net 3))
 (segment (start 139.87 72.4) (end 143.27 69) (width 0.2) (layer "B.Cu") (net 3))
 (segment (start 145.97 85.25) (end 145.399 84.679) (width 0.2) (layer "F.Cu") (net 1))
 (segment (start 144.819 86.401) (end 142.95324 86.401) (width 0.2) (layer "F.Cu") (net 1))
 (segment (start 145.399 84.679) (end 145.399 80.27101) (width 0.2) (layer "F.Cu") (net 1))
 (segment (start 149.151 78.19399) (end 149.151 77.47601) (width 0.2) (layer "F.Cu") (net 1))
 (segment (start 142.95324 86.401) (end 142.041 85.48876) (width 0.2) (layer "F.Cu") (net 1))
 (segment (start 149.151 77.47601) (end 148.23999 76.565) (width 0.2) (layer "F.Cu") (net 1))
 (segment (start 145.399 80.27101) (end 147.20901 78.461) (width 0.2) (layer "F.Cu") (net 1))
 (segment (start 139.13516 78.949) (end 137.551 78.949) (width 0.2) (layer "F.Cu") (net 1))
 (segment (start 142.041 85.48876) (end 142.041 81.85484) (width 0.2) (layer "F.Cu") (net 1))
 (segment (start 142.041 81.85484) (end 139.13516 78.949) (width 0.2) (layer "F.Cu") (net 1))
 (segment (start 137.551 78.949) (end 136.55 79.95) (width 0.2) (layer "F.Cu") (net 1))
 (segment (start 148.23999 76.565) (end 148.0375 76.565) (width 0.2) (layer "F.Cu") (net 1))
 (segment (start 148.88399 78.461) (end 149.151 78.19399) (width 0.2) (layer "F.Cu") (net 1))
 (segment (start 145.97 85.25) (end 144.819 86.401) (width 0.2) (layer "F.Cu") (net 1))
 (segment (start 147.20901 78.461) (end 148.88399 78.461) (width 0.2) (layer "F.Cu") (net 1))
 (segment (start 143.43 81.630001) (end 143.43 85.25) (width 0.2) (layer "F.Cu") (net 5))
 (segment (start 148.0375 77.835) (end 147.225001 77.835) (width 0.2) (layer "F.Cu") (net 5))
 (segment (start 143.65 80.85) (end 143.93 81.13) (width 0.2) (layer "F.Cu") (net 5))
 (segment (start 142.3 80.85) (end 143.65 80.85) (width 0.2) (layer "F.Cu") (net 5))
 (segment (start 138.4 77.75) (end 138.45 77.8) (width 0.2) (layer "F.Cu") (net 5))
 (segment (start 147.225001 77.835) (end 143.93 81.13) (width 0.2) (layer "F.Cu") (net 5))
 (segment (start 138.4 75.45) (end 138.4 77.75) (width 0.2) (layer "F.Cu") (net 5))
 (segment (start 143.93 81.13) (end 143.43 81.630001) (width 0.2) (layer "F.Cu") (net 5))
 (via (at 142.3 80.85) (size 0.6) (drill 0.3) (layers "F.Cu" "B.Cu") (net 5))
 (via (at 138.45 77.8) (size 0.6) (drill 0.3) (layers "F.Cu" "B.Cu") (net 5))
 (segment (start 138.45 77.8) (end 141.5 80.85) (width 0.2) (layer "B.Cu") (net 5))
 (segment (start 141.5 80.85) (end 142.3 80.85) (width 0.2) (layer "B.Cu") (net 5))
 (segment (start 148.0375 82.1625) (end 147.9 82.3) (width 0.2) (layer "F.Cu") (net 7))
 (segment (start 148.0375 79.105) (end 148.0375 82.1625) (width 0.2) (layer "F.Cu") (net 7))
 (via (at 147.9 82.3) (size 0.6) (drill 0.3) (layers "F.Cu" "B.Cu") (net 7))
 (segment (start 142.5 82.3) (end 140.89 83.91) (width 0.2) (layer "B.Cu") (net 7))
 (segment (start 140.89 83.91) (end 140.89 85.25) (width 0.2) (layer "B.Cu") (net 7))
 (segment (start 147.9 82.3) (end 142.5 82.3) (width 0.2) (layer "B.Cu") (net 7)))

